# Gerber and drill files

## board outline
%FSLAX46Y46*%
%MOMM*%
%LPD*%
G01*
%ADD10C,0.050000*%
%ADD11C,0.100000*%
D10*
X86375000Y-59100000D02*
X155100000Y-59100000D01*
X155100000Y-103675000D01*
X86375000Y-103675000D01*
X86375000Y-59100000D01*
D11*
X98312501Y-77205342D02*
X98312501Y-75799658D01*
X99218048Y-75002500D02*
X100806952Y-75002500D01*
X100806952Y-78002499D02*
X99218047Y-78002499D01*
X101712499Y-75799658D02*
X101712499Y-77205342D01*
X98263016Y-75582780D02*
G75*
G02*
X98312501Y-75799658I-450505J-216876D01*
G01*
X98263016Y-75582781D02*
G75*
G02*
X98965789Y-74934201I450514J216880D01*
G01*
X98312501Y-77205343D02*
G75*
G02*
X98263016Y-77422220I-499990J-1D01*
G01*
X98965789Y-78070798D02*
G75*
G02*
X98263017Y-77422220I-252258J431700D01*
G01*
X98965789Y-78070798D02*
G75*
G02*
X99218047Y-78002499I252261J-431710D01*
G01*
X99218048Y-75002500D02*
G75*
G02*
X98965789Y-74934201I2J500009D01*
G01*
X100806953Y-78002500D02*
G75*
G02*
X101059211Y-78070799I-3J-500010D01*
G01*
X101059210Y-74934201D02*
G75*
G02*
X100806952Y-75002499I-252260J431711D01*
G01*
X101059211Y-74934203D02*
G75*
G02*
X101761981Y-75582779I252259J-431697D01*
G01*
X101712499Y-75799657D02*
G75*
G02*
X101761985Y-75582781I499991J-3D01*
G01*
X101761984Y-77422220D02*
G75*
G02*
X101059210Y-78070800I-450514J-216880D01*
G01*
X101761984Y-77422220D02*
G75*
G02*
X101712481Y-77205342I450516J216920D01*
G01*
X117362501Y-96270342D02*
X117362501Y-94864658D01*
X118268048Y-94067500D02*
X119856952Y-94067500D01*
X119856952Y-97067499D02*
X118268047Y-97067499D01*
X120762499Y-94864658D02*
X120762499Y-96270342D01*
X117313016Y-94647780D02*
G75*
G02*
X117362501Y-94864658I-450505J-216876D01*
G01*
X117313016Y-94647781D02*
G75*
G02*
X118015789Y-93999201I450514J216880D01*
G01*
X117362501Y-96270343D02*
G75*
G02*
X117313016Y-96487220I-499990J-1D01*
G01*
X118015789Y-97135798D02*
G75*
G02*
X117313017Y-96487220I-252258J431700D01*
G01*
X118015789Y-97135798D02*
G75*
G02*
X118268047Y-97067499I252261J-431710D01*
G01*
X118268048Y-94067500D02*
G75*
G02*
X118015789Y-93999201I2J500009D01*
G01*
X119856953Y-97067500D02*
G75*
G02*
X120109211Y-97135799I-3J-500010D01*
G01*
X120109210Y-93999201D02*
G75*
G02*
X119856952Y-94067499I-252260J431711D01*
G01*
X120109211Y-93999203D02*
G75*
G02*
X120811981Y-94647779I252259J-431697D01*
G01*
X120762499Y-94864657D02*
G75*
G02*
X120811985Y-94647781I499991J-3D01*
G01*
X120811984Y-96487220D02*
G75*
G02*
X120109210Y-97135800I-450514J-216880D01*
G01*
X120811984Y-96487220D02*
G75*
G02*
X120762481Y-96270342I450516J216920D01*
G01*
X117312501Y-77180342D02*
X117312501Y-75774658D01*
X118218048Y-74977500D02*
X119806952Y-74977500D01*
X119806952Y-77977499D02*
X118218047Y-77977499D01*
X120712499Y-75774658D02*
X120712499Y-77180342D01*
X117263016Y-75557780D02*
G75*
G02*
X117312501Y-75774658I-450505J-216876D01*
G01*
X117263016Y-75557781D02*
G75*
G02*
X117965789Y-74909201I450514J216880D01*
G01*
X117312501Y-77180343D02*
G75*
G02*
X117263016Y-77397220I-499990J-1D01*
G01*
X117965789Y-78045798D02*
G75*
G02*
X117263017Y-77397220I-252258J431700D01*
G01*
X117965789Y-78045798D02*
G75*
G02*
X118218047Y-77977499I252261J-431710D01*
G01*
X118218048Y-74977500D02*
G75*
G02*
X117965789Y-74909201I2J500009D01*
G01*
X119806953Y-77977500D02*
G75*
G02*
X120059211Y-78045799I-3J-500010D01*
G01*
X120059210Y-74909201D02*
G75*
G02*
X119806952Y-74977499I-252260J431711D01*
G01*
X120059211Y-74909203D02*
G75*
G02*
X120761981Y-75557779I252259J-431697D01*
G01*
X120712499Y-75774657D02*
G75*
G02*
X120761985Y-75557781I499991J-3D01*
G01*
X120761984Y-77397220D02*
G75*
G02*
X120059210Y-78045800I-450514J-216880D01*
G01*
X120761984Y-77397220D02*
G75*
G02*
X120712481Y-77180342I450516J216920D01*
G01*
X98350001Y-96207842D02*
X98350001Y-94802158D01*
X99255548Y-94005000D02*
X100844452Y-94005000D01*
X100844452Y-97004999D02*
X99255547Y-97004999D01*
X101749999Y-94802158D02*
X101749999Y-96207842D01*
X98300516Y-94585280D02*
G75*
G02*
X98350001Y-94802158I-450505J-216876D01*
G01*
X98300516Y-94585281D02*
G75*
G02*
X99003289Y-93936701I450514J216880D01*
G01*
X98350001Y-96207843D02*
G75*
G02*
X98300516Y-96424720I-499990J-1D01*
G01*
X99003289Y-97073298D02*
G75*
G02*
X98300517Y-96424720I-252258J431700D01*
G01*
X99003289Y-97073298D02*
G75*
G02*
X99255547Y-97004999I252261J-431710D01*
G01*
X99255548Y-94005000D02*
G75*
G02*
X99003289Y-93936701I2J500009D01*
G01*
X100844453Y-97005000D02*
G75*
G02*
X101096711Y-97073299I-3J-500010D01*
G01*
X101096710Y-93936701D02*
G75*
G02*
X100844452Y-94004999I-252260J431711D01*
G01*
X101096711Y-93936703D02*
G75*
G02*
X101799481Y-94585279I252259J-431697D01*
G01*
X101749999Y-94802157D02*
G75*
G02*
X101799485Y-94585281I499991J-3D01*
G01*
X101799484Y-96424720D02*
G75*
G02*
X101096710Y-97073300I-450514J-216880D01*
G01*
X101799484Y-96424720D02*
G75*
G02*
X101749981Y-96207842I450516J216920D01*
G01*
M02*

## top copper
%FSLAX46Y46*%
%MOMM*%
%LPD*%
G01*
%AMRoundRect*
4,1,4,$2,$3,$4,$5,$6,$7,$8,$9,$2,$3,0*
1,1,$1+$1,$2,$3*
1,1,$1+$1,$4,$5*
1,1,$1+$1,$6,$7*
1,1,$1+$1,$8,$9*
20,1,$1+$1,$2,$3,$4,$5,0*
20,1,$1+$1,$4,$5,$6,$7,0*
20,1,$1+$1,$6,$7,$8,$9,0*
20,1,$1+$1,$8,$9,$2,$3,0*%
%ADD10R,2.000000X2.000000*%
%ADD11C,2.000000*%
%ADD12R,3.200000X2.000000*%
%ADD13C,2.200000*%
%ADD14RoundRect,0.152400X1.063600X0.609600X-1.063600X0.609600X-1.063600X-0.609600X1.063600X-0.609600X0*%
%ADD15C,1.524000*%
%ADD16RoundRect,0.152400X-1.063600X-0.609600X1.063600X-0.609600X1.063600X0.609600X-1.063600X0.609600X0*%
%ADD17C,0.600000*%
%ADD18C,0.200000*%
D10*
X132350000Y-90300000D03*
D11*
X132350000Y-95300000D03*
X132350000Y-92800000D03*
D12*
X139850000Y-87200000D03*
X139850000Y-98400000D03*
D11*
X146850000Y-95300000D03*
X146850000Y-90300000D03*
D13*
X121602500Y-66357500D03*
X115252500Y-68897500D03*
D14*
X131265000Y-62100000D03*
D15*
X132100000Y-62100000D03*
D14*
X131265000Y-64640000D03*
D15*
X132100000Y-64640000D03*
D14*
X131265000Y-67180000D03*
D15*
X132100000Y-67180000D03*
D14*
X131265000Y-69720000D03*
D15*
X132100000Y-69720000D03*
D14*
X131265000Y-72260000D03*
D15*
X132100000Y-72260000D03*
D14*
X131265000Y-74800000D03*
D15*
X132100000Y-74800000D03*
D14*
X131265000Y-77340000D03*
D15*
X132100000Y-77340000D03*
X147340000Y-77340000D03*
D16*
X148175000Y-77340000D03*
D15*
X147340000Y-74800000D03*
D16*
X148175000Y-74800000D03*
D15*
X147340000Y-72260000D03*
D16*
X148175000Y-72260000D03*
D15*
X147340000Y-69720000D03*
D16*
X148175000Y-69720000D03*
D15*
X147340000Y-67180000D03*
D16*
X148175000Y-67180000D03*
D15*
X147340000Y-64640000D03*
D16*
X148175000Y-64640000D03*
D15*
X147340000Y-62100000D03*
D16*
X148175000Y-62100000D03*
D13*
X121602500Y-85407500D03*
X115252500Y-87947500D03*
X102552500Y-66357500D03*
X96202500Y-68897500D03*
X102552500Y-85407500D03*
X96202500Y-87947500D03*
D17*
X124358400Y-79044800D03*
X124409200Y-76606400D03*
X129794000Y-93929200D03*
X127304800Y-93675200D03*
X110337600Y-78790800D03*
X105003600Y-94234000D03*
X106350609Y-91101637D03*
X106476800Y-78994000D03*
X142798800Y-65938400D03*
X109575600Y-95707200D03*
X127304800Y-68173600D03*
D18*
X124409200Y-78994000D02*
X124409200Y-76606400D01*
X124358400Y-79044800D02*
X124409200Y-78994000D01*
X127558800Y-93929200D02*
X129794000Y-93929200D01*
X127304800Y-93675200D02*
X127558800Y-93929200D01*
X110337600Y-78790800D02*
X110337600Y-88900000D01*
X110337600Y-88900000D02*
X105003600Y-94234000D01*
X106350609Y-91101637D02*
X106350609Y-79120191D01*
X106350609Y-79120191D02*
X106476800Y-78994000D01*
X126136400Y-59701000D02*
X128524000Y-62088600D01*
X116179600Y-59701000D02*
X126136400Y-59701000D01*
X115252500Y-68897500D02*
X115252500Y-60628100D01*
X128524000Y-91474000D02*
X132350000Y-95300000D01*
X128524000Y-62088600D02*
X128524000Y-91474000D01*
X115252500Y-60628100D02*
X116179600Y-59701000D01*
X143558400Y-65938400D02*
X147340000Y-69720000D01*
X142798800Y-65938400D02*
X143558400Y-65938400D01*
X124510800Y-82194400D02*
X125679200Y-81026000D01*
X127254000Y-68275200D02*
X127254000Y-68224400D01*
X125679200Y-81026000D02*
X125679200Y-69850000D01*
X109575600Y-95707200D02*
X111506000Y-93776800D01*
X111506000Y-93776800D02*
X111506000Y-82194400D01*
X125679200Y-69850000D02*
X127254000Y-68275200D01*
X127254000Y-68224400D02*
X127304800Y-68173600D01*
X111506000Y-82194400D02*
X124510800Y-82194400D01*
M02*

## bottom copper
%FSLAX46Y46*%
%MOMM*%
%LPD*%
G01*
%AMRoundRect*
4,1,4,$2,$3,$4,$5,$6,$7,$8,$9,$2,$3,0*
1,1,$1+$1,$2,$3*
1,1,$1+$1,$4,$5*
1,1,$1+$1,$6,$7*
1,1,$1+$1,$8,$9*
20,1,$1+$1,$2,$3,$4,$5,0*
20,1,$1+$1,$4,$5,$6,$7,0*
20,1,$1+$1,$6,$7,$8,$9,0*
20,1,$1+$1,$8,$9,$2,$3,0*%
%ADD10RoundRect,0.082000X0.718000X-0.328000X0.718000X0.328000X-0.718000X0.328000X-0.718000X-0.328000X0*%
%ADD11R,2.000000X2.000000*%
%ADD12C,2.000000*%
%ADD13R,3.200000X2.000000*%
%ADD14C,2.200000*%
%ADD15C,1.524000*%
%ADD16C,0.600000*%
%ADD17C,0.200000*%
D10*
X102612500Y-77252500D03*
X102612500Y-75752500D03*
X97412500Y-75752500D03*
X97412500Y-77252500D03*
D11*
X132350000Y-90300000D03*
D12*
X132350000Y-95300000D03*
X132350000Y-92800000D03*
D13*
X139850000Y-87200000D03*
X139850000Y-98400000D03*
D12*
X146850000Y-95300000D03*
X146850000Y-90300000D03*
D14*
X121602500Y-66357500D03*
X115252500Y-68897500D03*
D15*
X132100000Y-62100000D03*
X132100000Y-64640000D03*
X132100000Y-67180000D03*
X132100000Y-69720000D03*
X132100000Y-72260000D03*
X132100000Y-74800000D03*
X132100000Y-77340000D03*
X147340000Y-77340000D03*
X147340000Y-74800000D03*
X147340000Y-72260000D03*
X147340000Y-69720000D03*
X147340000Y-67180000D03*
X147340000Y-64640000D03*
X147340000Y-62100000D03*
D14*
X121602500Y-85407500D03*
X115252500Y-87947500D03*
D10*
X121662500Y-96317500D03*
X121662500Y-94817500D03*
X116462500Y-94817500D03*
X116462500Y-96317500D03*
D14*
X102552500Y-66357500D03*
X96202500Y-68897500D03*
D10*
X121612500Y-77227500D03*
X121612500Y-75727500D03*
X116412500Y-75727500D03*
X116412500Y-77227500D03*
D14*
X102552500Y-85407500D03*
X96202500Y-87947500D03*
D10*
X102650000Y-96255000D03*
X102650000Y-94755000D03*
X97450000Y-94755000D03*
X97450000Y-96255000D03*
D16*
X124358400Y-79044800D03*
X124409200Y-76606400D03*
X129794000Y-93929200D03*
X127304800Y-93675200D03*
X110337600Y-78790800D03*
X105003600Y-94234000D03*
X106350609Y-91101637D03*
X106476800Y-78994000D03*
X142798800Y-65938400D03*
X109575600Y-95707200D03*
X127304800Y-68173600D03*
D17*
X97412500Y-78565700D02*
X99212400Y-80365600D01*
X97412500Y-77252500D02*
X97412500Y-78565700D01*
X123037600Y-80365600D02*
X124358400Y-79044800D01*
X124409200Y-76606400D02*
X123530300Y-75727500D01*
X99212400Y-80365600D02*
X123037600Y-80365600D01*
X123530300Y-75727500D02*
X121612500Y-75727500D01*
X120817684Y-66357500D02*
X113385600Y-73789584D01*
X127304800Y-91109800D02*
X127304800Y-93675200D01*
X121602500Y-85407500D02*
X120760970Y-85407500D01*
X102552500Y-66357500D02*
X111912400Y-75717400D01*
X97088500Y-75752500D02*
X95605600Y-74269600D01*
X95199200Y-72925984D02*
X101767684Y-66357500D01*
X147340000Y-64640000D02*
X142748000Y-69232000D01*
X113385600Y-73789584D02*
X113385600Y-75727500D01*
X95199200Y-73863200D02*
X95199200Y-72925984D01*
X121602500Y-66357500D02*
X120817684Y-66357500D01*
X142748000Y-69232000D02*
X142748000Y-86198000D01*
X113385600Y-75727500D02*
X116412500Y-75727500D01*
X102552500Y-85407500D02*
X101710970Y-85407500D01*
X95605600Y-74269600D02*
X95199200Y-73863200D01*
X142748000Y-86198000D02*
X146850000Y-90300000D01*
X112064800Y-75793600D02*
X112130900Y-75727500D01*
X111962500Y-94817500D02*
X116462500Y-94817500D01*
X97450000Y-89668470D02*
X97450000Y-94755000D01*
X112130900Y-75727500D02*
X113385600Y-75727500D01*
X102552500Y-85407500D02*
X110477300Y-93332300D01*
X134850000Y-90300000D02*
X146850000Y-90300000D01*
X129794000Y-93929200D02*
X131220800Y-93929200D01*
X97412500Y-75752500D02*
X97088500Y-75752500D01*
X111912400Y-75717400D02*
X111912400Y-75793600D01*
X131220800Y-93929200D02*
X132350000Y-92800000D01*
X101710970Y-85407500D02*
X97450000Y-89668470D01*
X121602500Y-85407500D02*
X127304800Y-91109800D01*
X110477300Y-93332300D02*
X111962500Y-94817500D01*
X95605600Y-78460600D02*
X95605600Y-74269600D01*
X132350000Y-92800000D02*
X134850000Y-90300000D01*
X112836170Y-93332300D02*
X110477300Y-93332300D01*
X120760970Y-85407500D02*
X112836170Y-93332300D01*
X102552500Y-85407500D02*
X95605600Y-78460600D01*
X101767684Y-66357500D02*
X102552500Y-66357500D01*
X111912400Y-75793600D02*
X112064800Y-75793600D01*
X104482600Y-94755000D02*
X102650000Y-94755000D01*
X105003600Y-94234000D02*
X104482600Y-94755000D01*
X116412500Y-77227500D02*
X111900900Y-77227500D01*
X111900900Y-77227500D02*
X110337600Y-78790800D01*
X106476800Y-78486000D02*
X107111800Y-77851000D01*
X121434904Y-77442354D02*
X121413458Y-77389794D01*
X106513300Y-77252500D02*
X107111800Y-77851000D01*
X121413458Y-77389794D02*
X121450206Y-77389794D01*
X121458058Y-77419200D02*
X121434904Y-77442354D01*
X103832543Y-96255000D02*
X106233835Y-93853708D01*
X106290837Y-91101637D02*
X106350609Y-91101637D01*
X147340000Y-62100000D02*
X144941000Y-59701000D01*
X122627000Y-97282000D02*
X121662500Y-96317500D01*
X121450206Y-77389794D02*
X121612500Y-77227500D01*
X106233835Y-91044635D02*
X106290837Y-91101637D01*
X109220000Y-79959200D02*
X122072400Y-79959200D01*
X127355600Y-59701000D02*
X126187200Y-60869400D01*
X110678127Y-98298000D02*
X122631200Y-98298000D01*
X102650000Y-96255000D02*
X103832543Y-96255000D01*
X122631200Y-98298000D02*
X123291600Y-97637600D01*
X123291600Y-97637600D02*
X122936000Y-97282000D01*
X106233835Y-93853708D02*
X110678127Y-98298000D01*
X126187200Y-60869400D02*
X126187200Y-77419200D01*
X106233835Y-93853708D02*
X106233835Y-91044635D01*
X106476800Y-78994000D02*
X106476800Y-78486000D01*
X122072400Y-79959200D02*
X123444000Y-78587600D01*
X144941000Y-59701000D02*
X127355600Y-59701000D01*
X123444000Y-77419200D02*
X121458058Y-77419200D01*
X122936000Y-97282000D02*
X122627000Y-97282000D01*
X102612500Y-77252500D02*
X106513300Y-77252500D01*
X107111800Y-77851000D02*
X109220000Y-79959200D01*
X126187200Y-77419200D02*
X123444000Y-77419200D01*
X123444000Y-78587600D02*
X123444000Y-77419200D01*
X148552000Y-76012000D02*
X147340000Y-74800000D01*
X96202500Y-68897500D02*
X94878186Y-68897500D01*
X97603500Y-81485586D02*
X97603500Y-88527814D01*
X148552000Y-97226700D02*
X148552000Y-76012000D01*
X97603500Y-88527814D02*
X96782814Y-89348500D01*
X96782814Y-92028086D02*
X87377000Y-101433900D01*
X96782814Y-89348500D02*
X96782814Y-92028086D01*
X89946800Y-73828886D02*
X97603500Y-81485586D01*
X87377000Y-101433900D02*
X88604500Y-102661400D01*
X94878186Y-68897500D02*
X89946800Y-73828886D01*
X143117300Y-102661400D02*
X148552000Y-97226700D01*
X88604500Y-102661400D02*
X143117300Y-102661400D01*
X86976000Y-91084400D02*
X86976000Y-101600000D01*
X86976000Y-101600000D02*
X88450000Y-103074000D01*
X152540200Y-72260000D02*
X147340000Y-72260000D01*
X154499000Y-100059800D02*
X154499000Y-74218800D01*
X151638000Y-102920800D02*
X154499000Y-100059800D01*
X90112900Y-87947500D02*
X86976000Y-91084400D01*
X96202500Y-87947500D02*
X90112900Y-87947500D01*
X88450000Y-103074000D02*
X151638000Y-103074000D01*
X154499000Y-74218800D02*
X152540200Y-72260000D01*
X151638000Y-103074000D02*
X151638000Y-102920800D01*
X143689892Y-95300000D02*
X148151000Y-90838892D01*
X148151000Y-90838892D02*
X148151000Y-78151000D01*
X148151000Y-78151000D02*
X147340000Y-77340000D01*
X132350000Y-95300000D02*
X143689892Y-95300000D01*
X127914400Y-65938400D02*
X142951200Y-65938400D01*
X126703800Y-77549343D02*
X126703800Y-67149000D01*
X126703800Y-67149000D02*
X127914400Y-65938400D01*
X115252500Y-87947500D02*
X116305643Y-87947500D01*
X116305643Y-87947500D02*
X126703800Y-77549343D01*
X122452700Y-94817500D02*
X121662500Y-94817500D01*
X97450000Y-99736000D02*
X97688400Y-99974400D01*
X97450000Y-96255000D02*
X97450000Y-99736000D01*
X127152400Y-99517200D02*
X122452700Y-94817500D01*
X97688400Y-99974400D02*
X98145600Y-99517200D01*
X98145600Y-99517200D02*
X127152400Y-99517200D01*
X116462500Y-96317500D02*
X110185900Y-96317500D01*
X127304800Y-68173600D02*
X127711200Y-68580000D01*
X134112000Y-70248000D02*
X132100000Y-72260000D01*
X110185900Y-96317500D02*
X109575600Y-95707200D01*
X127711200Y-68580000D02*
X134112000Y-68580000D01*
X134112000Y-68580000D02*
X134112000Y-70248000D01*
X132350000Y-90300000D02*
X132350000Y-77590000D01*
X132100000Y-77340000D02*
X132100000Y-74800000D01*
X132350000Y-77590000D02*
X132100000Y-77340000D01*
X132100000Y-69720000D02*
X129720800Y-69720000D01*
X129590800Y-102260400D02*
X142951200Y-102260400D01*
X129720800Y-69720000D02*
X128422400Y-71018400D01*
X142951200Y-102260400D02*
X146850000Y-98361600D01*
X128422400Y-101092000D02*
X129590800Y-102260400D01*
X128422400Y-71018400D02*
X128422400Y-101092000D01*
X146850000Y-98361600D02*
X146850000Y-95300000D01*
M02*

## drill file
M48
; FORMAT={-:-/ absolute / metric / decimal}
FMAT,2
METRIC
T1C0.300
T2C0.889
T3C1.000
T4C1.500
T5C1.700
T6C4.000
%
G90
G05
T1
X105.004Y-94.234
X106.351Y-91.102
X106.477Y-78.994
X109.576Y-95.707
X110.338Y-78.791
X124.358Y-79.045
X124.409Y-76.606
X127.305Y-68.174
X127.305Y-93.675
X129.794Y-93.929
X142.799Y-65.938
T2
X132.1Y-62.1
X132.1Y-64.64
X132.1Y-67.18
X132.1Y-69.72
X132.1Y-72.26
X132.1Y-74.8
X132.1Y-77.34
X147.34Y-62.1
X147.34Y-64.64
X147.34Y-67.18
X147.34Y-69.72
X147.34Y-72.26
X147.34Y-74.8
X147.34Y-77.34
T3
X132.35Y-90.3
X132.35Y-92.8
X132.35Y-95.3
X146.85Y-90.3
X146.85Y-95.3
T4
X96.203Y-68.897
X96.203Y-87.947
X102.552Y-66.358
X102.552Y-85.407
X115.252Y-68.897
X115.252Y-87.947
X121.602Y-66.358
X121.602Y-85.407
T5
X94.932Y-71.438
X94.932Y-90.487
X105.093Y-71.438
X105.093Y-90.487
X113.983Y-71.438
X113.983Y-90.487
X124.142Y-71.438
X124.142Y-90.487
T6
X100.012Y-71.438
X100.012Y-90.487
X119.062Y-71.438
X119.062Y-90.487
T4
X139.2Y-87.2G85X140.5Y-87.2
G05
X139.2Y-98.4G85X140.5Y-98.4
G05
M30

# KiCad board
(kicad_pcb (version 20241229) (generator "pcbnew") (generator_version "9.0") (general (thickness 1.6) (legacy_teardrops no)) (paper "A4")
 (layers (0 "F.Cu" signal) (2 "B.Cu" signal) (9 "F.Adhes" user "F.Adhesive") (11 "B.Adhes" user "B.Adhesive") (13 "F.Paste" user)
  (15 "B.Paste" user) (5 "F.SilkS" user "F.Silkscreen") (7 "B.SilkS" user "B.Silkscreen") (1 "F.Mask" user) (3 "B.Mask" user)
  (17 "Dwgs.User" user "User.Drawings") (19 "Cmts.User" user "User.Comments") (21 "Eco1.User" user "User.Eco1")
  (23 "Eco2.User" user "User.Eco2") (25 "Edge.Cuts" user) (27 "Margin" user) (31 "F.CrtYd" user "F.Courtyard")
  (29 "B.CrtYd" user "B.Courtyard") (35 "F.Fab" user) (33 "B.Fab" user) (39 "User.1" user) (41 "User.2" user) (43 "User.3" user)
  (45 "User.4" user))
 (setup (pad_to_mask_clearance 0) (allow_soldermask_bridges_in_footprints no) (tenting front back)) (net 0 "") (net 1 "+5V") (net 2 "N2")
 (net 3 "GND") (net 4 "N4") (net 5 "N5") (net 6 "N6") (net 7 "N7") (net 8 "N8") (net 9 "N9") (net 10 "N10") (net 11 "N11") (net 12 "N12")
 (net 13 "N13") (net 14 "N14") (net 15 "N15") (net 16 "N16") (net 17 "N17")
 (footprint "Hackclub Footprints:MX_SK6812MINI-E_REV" (layer "F.Cu") (at 100.0125 71.4225)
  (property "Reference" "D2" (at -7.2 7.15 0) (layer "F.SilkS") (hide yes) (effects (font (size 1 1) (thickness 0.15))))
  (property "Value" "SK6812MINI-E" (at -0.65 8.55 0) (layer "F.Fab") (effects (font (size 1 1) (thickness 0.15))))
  (fp_line (start -1.699999 5.782842) (end -1.699999 4.377158) (stroke (width 0.1) (type solid)) (layer "Edge.Cuts"))
  (fp_line (start -0.794452 3.58) (end 0.794452 3.58) (stroke (width 0.1) (type solid)) (layer "Edge.Cuts"))
  (fp_line (start 0.794452 6.579999) (end -0.794453 6.579999) (stroke (width 0.1) (type solid)) (layer "Edge.Cuts"))
  (fp_line (start 1.699999 4.377158) (end 1.699999 5.782842) (stroke (width 0.1) (type solid)) (layer "Edge.Cuts"))
  (fp_arc (start -1.749484 4.16028) (mid -1.712527 4.265932) (end -1.699999 4.377158) (stroke (width 0.1) (type solid)) (layer "Edge.Cuts"))
  (fp_arc (start -1.749484 4.160281) (mid -1.638072 3.575965) (end -1.046711 3.511701) (stroke (width 0.1) (type solid)) (layer "Edge.Cuts"))
  (fp_arc (start -1.699999 5.782843) (mid -1.712527 5.894068) (end -1.749484 5.99972) (stroke (width 0.1) (type solid)) (layer "Edge.Cuts"))
  (fp_arc (start -1.046711 6.648298) (mid -1.638071 6.584034) (end -1.749484 5.99972) (stroke (width 0.1) (type solid)) (layer "Edge.Cuts"))
  (fp_arc (start -1.046711 6.648298) (mid -0.925123 6.597376) (end -0.794453 6.579999) (stroke (width 0.1) (type solid)) (layer "Edge.Cuts"))
  (fp_arc (start -0.794452 3.58) (mid -0.925123 3.562623) (end -1.046711 3.511701) (stroke (width 0.1) (type solid)) (layer "Edge.Cuts"))
  (fp_arc (start 0.794453 6.58) (mid 0.925123 6.597377) (end 1.046711 6.648299) (stroke (width 0.1) (type solid)) (layer "Edge.Cuts"))
  (fp_arc (start 1.04671 3.511701) (mid 0.925122 3.562623) (end 0.794452 3.58) (stroke (width 0.1) (type solid)) (layer "Edge.Cuts"))
  (fp_arc (start 1.046711 3.511703) (mid 1.63807 3.575966) (end 1.749484 4.16028) (stroke (width 0.1) (type solid)) (layer "Edge.Cuts"))
  (fp_arc (start 1.699999 4.377157) (mid 1.712527 4.265932) (end 1.749484 4.16028) (stroke (width 0.1) (type solid)) (layer "Edge.Cuts"))
  (fp_arc (start 1.749484 5.99972) (mid 1.638071 6.584035) (end 1.046711 6.648299) (stroke (width 0.1) (type solid)) (layer "Edge.Cuts"))
  (fp_arc (start 1.749484 5.99972) (mid 1.712527 5.894068) (end 1.699999 5.782842) (stroke (width 0.1) (type solid)) (layer "Edge.Cuts"))
  (pad "1" smd roundrect (at 2.6 5.83 90) (size 0.82 1.6) (layers "B.Cu" "B.Mask" "B.Paste") (roundrect_rratio 0.1) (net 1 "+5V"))
  (pad "2" smd roundrect (at 2.6 4.33 90) (size 0.82 1.6) (layers "B.Cu" "B.Mask" "B.Paste") (roundrect_rratio 0.1) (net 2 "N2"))
  (pad "3" smd roundrect (at -2.6 4.33 90) (size 0.82 1.6) (layers "B.Cu" "B.Mask" "B.Paste") (roundrect_rratio 0.1) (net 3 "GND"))
  (pad "4" smd roundrect (at -2.6 5.83 90) (size 0.82 1.6) (layers "B.Cu" "B.Mask" "B.Paste") (roundrect_rratio 0.1) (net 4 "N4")))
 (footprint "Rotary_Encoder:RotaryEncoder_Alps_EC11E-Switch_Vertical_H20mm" (layer "F.Cu") (at 132.35 90.3)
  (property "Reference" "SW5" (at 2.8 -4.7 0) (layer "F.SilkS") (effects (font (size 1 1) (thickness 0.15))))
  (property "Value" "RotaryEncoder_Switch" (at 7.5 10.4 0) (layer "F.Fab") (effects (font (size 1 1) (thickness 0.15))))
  (pad "A" thru_hole rect (at 0 0) (size 2 2) (drill 1) (layers "*.Cu" "*.Mask") (remove_unused_layers no) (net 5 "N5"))
  (pad "B" thru_hole circle (at 0 5) (size 2 2) (drill 1) (layers "*.Cu" "*.Mask") (remove_unused_layers no) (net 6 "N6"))
  (pad "C" thru_hole circle (at 0 2.5) (size 2 2) (drill 1) (layers "*.Cu" "*.Mask") (remove_unused_layers no) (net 3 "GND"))
  (pad "MP" thru_hole rect (at 7.5 -3.1) (size 3.2 2) (drill oval 2.8 1.5) (layers "*.Cu" "*.Mask") (remove_unused_layers no))
  (pad "MP" thru_hole rect (at 7.5 8.1) (size 3.2 2) (drill oval 2.8 1.5) (layers "*.Cu" "*.Mask") (remove_unused_layers no))
  (pad "S1" thru_hole circle (at 14.5 5) (size 2 2) (drill 1) (layers "*.Cu" "*.Mask") (remove_unused_layers no) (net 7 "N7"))
  (pad "S2" thru_hole circle (at 14.5 0) (size 2 2) (drill 1) (layers "*.Cu" "*.Mask") (remove_unused_layers no) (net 3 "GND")))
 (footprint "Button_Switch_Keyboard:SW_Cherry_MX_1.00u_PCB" (layer "F.Cu") (at 121.6025 66.3575)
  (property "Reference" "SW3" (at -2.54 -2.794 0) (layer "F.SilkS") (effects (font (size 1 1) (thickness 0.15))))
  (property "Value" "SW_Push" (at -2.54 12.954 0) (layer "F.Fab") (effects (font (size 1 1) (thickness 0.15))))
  (pad "" np_thru_hole circle (at -7.62 5.08) (size 1.7 1.7) (drill 1.7) (layers "*.Cu" "*.Mask"))
  (pad "" np_thru_hole circle (at -2.54 5.08) (size 4 4) (drill 4) (layers "*.Cu" "*.Mask"))
  (pad "" np_thru_hole circle (at 2.54 5.08) (size 1.7 1.7) (drill 1.7) (layers "*.Cu" "*.Mask"))
  (pad "1" thru_hole circle (at 0 0) (size 2.2 2.2) (drill 1.5) (layers "*.Cu" "*.Mask") (remove_unused_layers no) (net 3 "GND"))
  (pad "2" thru_hole circle (at -6.35 2.54) (size 2.2 2.2) (drill 1.5) (layers "*.Cu" "*.Mask") (remove_unused_layers no) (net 6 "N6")))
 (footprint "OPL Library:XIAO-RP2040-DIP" (layer "F.Cu") (at 139.72 69.72)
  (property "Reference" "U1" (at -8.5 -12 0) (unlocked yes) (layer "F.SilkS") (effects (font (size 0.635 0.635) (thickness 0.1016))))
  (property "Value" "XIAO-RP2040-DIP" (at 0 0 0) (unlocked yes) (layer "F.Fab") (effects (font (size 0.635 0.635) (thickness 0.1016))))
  (pad "1" smd roundrect (at -8.455 -7.62 180) (size 2.432 1.524) (layers "F.Cu" "F.Mask") (roundrect_rratio 0.1) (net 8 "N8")
   (thermal_bridge_angle 45))
  (pad "1" thru_hole circle (at -7.62 -7.62 180) (size 1.524 1.524) (drill 0.889) (layers "*.Cu" "*.Mask") (remove_unused_layers no)
   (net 8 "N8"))
  (pad "2" smd roundrect (at -8.455 -5.08 180) (size 2.432 1.524) (layers "F.Cu" "F.Mask") (roundrect_rratio 0.1) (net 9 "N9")
   (thermal_bridge_angle 45))
  (pad "2" thru_hole circle (at -7.62 -5.08 180) (size 1.524 1.524) (drill 0.889) (layers "*.Cu" "*.Mask") (remove_unused_layers no)
   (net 9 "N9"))
  (pad "3" smd roundrect (at -8.455 -2.54 180) (size 2.432 1.524) (layers "F.Cu" "F.Mask") (roundrect_rratio 0.1) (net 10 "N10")
   (thermal_bridge_angle 45))
  (pad "3" thru_hole circle (at -7.62 -2.54 180) (size 1.524 1.524) (drill 0.889) (layers "*.Cu" "*.Mask") (remove_unused_layers no)
   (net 10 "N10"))
  (pad "4" smd roundrect (at -8.455 0 180) (size 2.432 1.524) (layers "F.Cu" "F.Mask") (roundrect_rratio 0.1) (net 7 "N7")
   (thermal_bridge_angle 45))
  (pad "4" thru_hole circle (at -7.62 0 180) (size 1.524 1.524) (drill 0.889) (layers "*.Cu" "*.Mask") (remove_unused_layers no)
   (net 7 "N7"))
  (pad "5" smd roundrect (at -8.455 2.54 180) (size 2.432 1.524) (layers "F.Cu" "F.Mask") (roundrect_rratio 0.1) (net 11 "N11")
   (thermal_bridge_angle 45))
  (pad "5" thru_hole circle (at -7.62 2.54 180) (size 1.524 1.524) (drill 0.889) (layers "*.Cu" "*.Mask") (remove_unused_layers no)
   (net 11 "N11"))
  (pad "6" smd roundrect (at -8.455 5.08 180) (size 2.432 1.524) (layers "F.Cu" "F.Mask") (roundrect_rratio 0.1) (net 5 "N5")
   (thermal_bridge_angle 45))
  (pad "6" thru_hole circle (at -7.62 5.08 180) (size 1.524 1.524) (drill 0.889) (layers "*.Cu" "*.Mask") (remove_unused_layers no)
   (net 5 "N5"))
  (pad "7" smd roundrect (at -8.455 7.62 180) (size 2.432 1.524) (layers "F.Cu" "F.Mask") (roundrect_rratio 0.1) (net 5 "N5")
   (thermal_bridge_angle 45))
  (pad "7" thru_hole circle (at -7.62 7.62 180) (size 1.524 1.524) (drill 0.889) (layers "*.Cu" "*.Mask") (remove_unused_layers no)
   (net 5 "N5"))
  (pad "8" thru_hole circle (at 7.62 7.62) (size 1.524 1.524) (drill 0.889) (layers "*.Cu" "*.Mask") (remove_unused_layers no) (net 6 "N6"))
  (pad "8" smd roundrect (at 8.455 7.62) (size 2.432 1.524) (layers "F.Cu" "F.Mask") (roundrect_rratio 0.1) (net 6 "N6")
   (thermal_bridge_angle 45))
  (pad "9" thru_hole circle (at 7.62 5.08) (size 1.524 1.524) (drill 0.889) (layers "*.Cu" "*.Mask") (remove_unused_layers no)
   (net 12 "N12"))
  (pad "9" smd roundrect (at 8.455 5.08) (size 2.432 1.524) (layers "F.Cu" "F.Mask") (roundrect_rratio 0.1) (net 12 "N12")
   (thermal_bridge_angle 45))
  (pad "10" thru_hole circle (at 7.62 2.54) (size 1.524 1.524) (drill 0.889) (layers "*.Cu" "*.Mask") (remove_unused_layers no)
   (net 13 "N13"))
  (pad "10" smd roundrect (at 8.455 2.54) (size 2.432 1.524) (layers "F.Cu" "F.Mask") (roundrect_rratio 0.1) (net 13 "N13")
   (thermal_bridge_angle 45))
  (pad "11" thru_hole circle (at 7.62 0) (size 1.524 1.524) (drill 0.889) (layers "*.Cu" "*.Mask") (remove_unused_layers no) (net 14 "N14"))
  (pad "11" smd roundrect (at 8.455 0) (size 2.432 1.524) (layers "F.Cu" "F.Mask") (roundrect_rratio 0.1) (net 14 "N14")
   (thermal_bridge_angle 45))
  (pad "12" thru_hole circle (at 7.62 -2.54) (size 1.524 1.524) (drill 0.889) (layers "*.Cu" "*.Mask") (remove_unused_layers no)
   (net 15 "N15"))
  (pad "12" smd roundrect (at 8.455 -2.54) (size 2.432 1.524) (layers "F.Cu" "F.Mask") (roundrect_rratio 0.1) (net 15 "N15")
   (thermal_bridge_angle 45))
  (pad "13" thru_hole circle (at 7.62 -5.08) (size 1.524 1.524) (drill 0.889) (layers "*.Cu" "*.Mask") (remove_unused_layers no)
   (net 3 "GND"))
  (pad "13" smd roundrect (at 8.455 -5.08) (size 2.432 1.524) (layers "F.Cu" "F.Mask") (roundrect_rratio 0.1) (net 3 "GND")
   (thermal_bridge_angle 45))
  (pad "14" thru_hole circle (at 7.62 -7.62) (size 1.524 1.524) (drill 0.889) (layers "*.Cu" "*.Mask") (remove_unused_layers no)
   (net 1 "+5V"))
  (pad "14" smd roundrect (at 8.455 -7.62) (size 2.432 1.524) (layers "F.Cu" "F.Mask") (roundrect_rratio 0.1) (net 1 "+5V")
   (thermal_bridge_angle 45)))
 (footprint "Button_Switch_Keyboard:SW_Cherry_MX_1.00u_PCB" (layer "F.Cu") (at 121.6025 85.4075)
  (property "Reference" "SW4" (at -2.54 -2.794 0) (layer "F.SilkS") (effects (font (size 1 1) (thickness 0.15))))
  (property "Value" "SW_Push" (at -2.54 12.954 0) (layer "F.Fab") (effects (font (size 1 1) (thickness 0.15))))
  (pad "" np_thru_hole circle (at -7.62 5.08) (size 1.7 1.7) (drill 1.7) (layers "*.Cu" "*.Mask"))
  (pad "" np_thru_hole circle (at -2.54 5.08) (size 4 4) (drill 4) (layers "*.Cu" "*.Mask"))
  (pad "" np_thru_hole circle (at 2.54 5.08) (size 1.7 1.7) (drill 1.7) (layers "*.Cu" "*.Mask"))
  (pad "1" thru_hole circle (at 0 0) (size 2.2 2.2) (drill 1.5) (layers "*.Cu" "*.Mask") (remove_unused_layers no) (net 3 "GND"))
  (pad "2" thru_hole circle (at -6.35 2.54) (size 2.2 2.2) (drill 1.5) (layers "*.Cu" "*.Mask") (remove_unused_layers no) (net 14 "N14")))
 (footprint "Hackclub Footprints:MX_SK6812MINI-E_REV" (layer "F.Cu") (at 119.0625 90.4875)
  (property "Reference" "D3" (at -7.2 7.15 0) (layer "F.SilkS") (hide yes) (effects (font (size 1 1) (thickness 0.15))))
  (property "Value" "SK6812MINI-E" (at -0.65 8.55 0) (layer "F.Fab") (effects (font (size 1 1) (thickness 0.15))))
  (fp_line (start -1.699999 5.782842) (end -1.699999 4.377158) (stroke (width 0.1) (type solid)) (layer "Edge.Cuts"))
  (fp_line (start -0.794452 3.58) (end 0.794452 3.58) (stroke (width 0.1) (type solid)) (layer "Edge.Cuts"))
  (fp_line (start 0.794452 6.579999) (end -0.794453 6.579999) (stroke (width 0.1) (type solid)) (layer "Edge.Cuts"))
  (fp_line (start 1.699999 4.377158) (end 1.699999 5.782842) (stroke (width 0.1) (type solid)) (layer "Edge.Cuts"))
  (fp_arc (start -1.749484 4.16028) (mid -1.712527 4.265932) (end -1.699999 4.377158) (stroke (width 0.1) (type solid)) (layer "Edge.Cuts"))
  (fp_arc (start -1.749484 4.160281) (mid -1.638072 3.575965) (end -1.046711 3.511701) (stroke (width 0.1) (type solid)) (layer "Edge.Cuts"))
  (fp_arc (start -1.699999 5.782843) (mid -1.712527 5.894068) (end -1.749484 5.99972) (stroke (width 0.1) (type solid)) (layer "Edge.Cuts"))
  (fp_arc (start -1.046711 6.648298) (mid -1.638071 6.584034) (end -1.749484 5.99972) (stroke (width 0.1) (type solid)) (layer "Edge.Cuts"))
  (fp_arc (start -1.046711 6.648298) (mid -0.925123 6.597376) (end -0.794453 6.579999) (stroke (width 0.1) (type solid)) (layer "Edge.Cuts"))
  (fp_arc (start -0.794452 3.58) (mid -0.925123 3.562623) (end -1.046711 3.511701) (stroke (width 0.1) (type solid)) (layer "Edge.Cuts"))
  (fp_arc (start 0.794453 6.58) (mid 0.925123 6.597377) (end 1.046711 6.648299) (stroke (width 0.1) (type solid)) (layer "Edge.Cuts"))
  (fp_arc (start 1.04671 3.511701) (mid 0.925122 3.562623) (end 0.794452 3.58) (stroke (width 0.1) (type solid)) (layer "Edge.Cuts"))
  (fp_arc (start 1.046711 3.511703) (mid 1.63807 3.575966) (end 1.749484 4.16028) (stroke (width 0.1) (type solid)) (layer "Edge.Cuts"))
  (fp_arc (start 1.699999 4.377157) (mid 1.712527 4.265932) (end 1.749484 4.16028) (stroke (width 0.1) (type solid)) (layer "Edge.Cuts"))
  (fp_arc (start 1.749484 5.99972) (mid 1.638071 6.584035) (end 1.046711 6.648299) (stroke (width 0.1) (type solid)) (layer "Edge.Cuts"))
  (fp_arc (start 1.749484 5.99972) (mid 1.712527 5.894068) (end 1.699999 5.782842) (stroke (width 0.1) (type solid)) (layer "Edge.Cuts"))
  (pad "1" smd roundrect (at 2.6 5.83 90) (size 0.82 1.6) (layers "B.Cu" "B.Mask" "B.Paste") (roundrect_rratio 0.1) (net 1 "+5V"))
  (pad "2" smd roundrect (at 2.6 4.33 90) (size 0.82 1.6) (layers "B.Cu" "B.Mask" "B.Paste") (roundrect_rratio 0.1) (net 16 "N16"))
  (pad "3" smd roundrect (at -2.6 4.33 90) (size 0.82 1.6) (layers "B.Cu" "B.Mask" "B.Paste") (roundrect_rratio 0.1) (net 3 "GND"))
  (pad "4" smd roundrect (at -2.6 5.83 90) (size 0.82 1.6) (layers "B.Cu" "B.Mask" "B.Paste") (roundrect_rratio 0.1) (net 11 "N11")))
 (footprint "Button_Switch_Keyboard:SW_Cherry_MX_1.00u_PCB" (layer "F.Cu") (at 102.5525 66.3575)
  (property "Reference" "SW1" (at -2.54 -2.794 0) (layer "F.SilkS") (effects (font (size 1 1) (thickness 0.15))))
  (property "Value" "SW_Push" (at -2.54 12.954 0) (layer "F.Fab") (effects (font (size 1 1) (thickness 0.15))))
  (pad "" np_thru_hole circle (at -7.62 5.08) (size 1.7 1.7) (drill 1.7) (layers "*.Cu" "*.Mask"))
  (pad "" np_thru_hole circle (at -2.54 5.08) (size 4 4) (drill 4) (layers "*.Cu" "*.Mask"))
  (pad "" np_thru_hole circle (at 2.54 5.08) (size 1.7 1.7) (drill 1.7) (layers "*.Cu" "*.Mask"))
  (pad "1" thru_hole circle (at 0 0) (size 2.2 2.2) (drill 1.5) (layers "*.Cu" "*.Mask") (remove_unused_layers no) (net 3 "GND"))
  (pad "2" thru_hole circle (at -6.35 2.54) (size 2.2 2.2) (drill 1.5) (layers "*.Cu" "*.Mask") (remove_unused_layers no) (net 12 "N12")))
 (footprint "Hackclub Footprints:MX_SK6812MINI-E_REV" (layer "F.Cu") (at 119.0125 71.3975)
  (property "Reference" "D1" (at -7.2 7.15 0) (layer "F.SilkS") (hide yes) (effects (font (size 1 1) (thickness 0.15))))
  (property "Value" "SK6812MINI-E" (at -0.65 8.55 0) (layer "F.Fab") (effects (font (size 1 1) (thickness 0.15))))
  (fp_line (start -1.699999 5.782842) (end -1.699999 4.377158) (stroke (width 0.1) (type solid)) (layer "Edge.Cuts"))
  (fp_line (start -0.794452 3.58) (end 0.794452 3.58) (stroke (width 0.1) (type solid)) (layer "Edge.Cuts"))
  (fp_line (start 0.794452 6.579999) (end -0.794453 6.579999) (stroke (width 0.1) (type solid)) (layer "Edge.Cuts"))
  (fp_line (start 1.699999 4.377158) (end 1.699999 5.782842) (stroke (width 0.1) (type solid)) (layer "Edge.Cuts"))
  (fp_arc (start -1.749484 4.16028) (mid -1.712527 4.265932) (end -1.699999 4.377158) (stroke (width 0.1) (type solid)) (layer "Edge.Cuts"))
  (fp_arc (start -1.749484 4.160281) (mid -1.638072 3.575965) (end -1.046711 3.511701) (stroke (width 0.1) (type solid)) (layer "Edge.Cuts"))
  (fp_arc (start -1.699999 5.782843) (mid -1.712527 5.894068) (end -1.749484 5.99972) (stroke (width 0.1) (type solid)) (layer "Edge.Cuts"))
  (fp_arc (start -1.046711 6.648298) (mid -1.638071 6.584034) (end -1.749484 5.99972) (stroke (width 0.1) (type solid)) (layer "Edge.Cuts"))
  (fp_arc (start -1.046711 6.648298) (mid -0.925123 6.597376) (end -0.794453 6.579999) (stroke (width 0.1) (type solid)) (layer "Edge.Cuts"))
  (fp_arc (start -0.794452 3.58) (mid -0.925123 3.562623) (end -1.046711 3.511701) (stroke (width 0.1) (type solid)) (layer "Edge.Cuts"))
  (fp_arc (start 0.794453 6.58) (mid 0.925123 6.597377) (end 1.046711 6.648299) (stroke (width 0.1) (type solid)) (layer "Edge.Cuts"))
  (fp_arc (start 1.04671 3.511701) (mid 0.925122 3.562623) (end 0.794452 3.58) (stroke (width 0.1) (type solid)) (layer "Edge.Cuts"))
  (fp_arc (start 1.046711 3.511703) (mid 1.63807 3.575966) (end 1.749484 4.16028) (stroke (width 0.1) (type solid)) (layer "Edge.Cuts"))
  (fp_arc (start 1.699999 4.377157) (mid 1.712527 4.265932) (end 1.749484 4.16028) (stroke (width 0.1) (type solid)) (layer "Edge.Cuts"))
  (fp_arc (start 1.749484 5.99972) (mid 1.638071 6.584035) (end 1.046711 6.648299) (stroke (width 0.1) (type solid)) (layer "Edge.Cuts"))
  (fp_arc (start 1.749484 5.99972) (mid 1.712527 5.894068) (end 1.699999 5.782842) (stroke (width 0.1) (type solid)) (layer "Edge.Cuts"))
  (pad "1" smd roundrect (at 2.6 5.83 90) (size 0.82 1.6) (layers "B.Cu" "B.Mask" "B.Paste") (roundrect_rratio 0.1) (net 1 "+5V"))
  (pad "2" smd roundrect (at 2.6 4.33 90) (size 0.82 1.6) (layers "B.Cu" "B.Mask" "B.Paste") (roundrect_rratio 0.1) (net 4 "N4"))
  (pad "3" smd roundrect (at -2.6 4.33 90) (size 0.82 1.6) (layers "B.Cu" "B.Mask" "B.Paste") (roundrect_rratio 0.1) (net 3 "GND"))
  (pad "4" smd roundrect (at -2.6 5.83 90) (size 0.82 1.6) (layers "B.Cu" "B.Mask" "B.Paste") (roundrect_rratio 0.1) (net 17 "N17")))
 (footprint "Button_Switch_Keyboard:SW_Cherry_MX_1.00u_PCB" (layer "F.Cu") (at 102.5525 85.4075)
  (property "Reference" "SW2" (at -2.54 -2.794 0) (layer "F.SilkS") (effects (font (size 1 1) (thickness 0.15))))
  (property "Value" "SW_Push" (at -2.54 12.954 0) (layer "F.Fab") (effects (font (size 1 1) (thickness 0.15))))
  (pad "" np_thru_hole circle (at -7.62 5.08) (size 1.7 1.7) (drill 1.7) (layers "*.Cu" "*.Mask"))
  (pad "" np_thru_hole circle (at -2.54 5.08) (size 4 4) (drill 4) (layers "*.Cu" "*.Mask"))
  (pad "" np_thru_hole circle (at 2.54 5.08) (size 1.7 1.7) (drill 1.7) (layers "*.Cu" "*.Mask"))
  (pad "1" thru_hole circle (at 0 0) (size 2.2 2.2) (drill 1.5) (layers "*.Cu" "*.Mask") (remove_unused_layers no) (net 3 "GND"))
  (pad "2" thru_hole circle (at -6.35 2.54) (size 2.2 2.2) (drill 1.5) (layers "*.Cu" "*.Mask") (remove_unused_layers no) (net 13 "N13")))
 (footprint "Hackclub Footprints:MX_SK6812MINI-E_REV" (layer "F.Cu") (at 100.05 90.425)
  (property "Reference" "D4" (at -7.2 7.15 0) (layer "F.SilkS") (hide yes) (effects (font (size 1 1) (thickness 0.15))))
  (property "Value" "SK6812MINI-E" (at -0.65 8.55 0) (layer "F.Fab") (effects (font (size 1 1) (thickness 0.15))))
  (fp_line (start -1.699999 5.782842) (end -1.699999 4.377158) (stroke (width 0.1) (type solid)) (layer "Edge.Cuts"))
  (fp_line (start -0.794452 3.58) (end 0.794452 3.58) (stroke (width 0.1) (type solid)) (layer "Edge.Cuts"))
  (fp_line (start 0.794452 6.579999) (end -0.794453 6.579999) (stroke (width 0.1) (type solid)) (layer "Edge.Cuts"))
  (fp_line (start 1.699999 4.377158) (end 1.699999 5.782842) (stroke (width 0.1) (type solid)) (layer "Edge.Cuts"))
  (fp_arc (start -1.749484 4.16028) (mid -1.712527 4.265932) (end -1.699999 4.377158) (stroke (width 0.1) (type solid)) (layer "Edge.Cuts"))
  (fp_arc (start -1.749484 4.160281) (mid -1.638072 3.575965) (end -1.046711 3.511701) (stroke (width 0.1) (type solid)) (layer "Edge.Cuts"))
  (fp_arc (start -1.699999 5.782843) (mid -1.712527 5.894068) (end -1.749484 5.99972) (stroke (width 0.1) (type solid)) (layer "Edge.Cuts"))
  (fp_arc (start -1.046711 6.648298) (mid -1.638071 6.584034) (end -1.749484 5.99972) (stroke (width 0.1) (type solid)) (layer "Edge.Cuts"))
  (fp_arc (start -1.046711 6.648298) (mid -0.925123 6.597376) (end -0.794453 6.579999) (stroke (width 0.1) (type solid)) (layer "Edge.Cuts"))
  (fp_arc (start -0.794452 3.58) (mid -0.925123 3.562623) (end -1.046711 3.511701) (stroke (width 0.1) (type solid)) (layer "Edge.Cuts"))
  (fp_arc (start 0.794453 6.58) (mid 0.925123 6.597377) (end 1.046711 6.648299) (stroke (width 0.1) (type solid)) (layer "Edge.Cuts"))
  (fp_arc (start 1.04671 3.511701) (mid 0.925122 3.562623) (end 0.794452 3.58) (stroke (width 0.1) (type solid)) (layer "Edge.Cuts"))
  (fp_arc (start 1.046711 3.511703) (mid 1.63807 3.575966) (end 1.749484 4.16028) (stroke (width 0.1) (type solid)) (layer "Edge.Cuts"))
  (fp_arc (start 1.699999 4.377157) (mid 1.712527 4.265932) (end 1.749484 4.16028) (stroke (width 0.1) (type solid)) (layer "Edge.Cuts"))
  (fp_arc (start 1.749484 5.99972) (mid 1.638071 6.584035) (end 1.046711 6.648299) (stroke (width 0.1) (type solid)) (layer "Edge.Cuts"))
  (fp_arc (start 1.749484 5.99972) (mid 1.712527 5.894068) (end 1.699999 5.782842) (stroke (width 0.1) (type solid)) (layer "Edge.Cuts"))
  (pad "1" smd roundrect (at 2.6 5.83 90) (size 0.82 1.6) (layers "B.Cu" "B.Mask" "B.Paste") (roundrect_rratio 0.1) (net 1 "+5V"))
  (pad "2" smd roundrect (at 2.6 4.33 90) (size 0.82 1.6) (layers "B.Cu" "B.Mask" "B.Paste") (roundrect_rratio 0.1) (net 17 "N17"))
  (pad "3" smd roundrect (at -2.6 4.33 90) (size 0.82 1.6) (layers "B.Cu" "B.Mask" "B.Paste") (roundrect_rratio 0.1) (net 3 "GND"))
  (pad "4" smd roundrect (at -2.6 5.83 90) (size 0.82 1.6) (layers "B.Cu" "B.Mask" "B.Paste") (roundrect_rratio 0.1) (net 16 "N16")))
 (gr_rect (start 86.375 59.1) (end 155.1 103.675) (stroke (width 0.05) (type default)) (fill no) (layer "Edge.Cuts"))
 (segment (start 124.4092 78.994) (end 124.4092 76.6064) (width 0.2) (layer "F.Cu") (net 4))
 (segment (start 124.3584 79.0448) (end 124.4092 78.994) (width 0.2) (layer "F.Cu") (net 4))
 (via (at 124.3584 79.0448) (size 0.6) (drill 0.3) (layers "F.Cu" "B.Cu") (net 4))
 (via (at 124.4092 76.6064) (size 0.6) (drill 0.3) (layers "F.Cu" "B.Cu") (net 4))
 (segment (start 97.4125 78.5657) (end 99.2124 80.3656) (width 0.2) (layer "B.Cu") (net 4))
 (segment (start 97.4125 77.2525) (end 97.4125 78.5657) (width 0.2) (layer "B.Cu") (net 4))
 (segment (start 123.0376 80.3656) (end 124.3584 79.0448) (width 0.2) (layer "B.Cu") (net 4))
 (segment (start 124.4092 76.6064) (end 123.5303 75.7275) (width 0.2) (layer "B.Cu") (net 4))
 (segment (start 99.2124 80.3656) (end 123.0376 80.3656) (width 0.2) (layer "B.Cu") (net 4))
 (segment (start 123.5303 75.7275) (end 121.6125 75.7275) (width 0.2) (layer "B.Cu") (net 4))
 (segment (start 127.5588 93.9292) (end 129.794 93.9292) (width 0.2) (layer "F.Cu") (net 3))
 (segment (start 127.3048 93.6752) (end 127.5588 93.9292) (width 0.2) (layer "F.Cu") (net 3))
 (via (at 129.794 93.9292) (size 0.6) (drill 0.3) (layers "F.Cu" "B.Cu") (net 3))
 (via (at 127.3048 93.6752) (size 0.6) (drill 0.3) (layers "F.Cu" "B.Cu") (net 3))
 (segment (start 120.817684 66.3575) (end 113.3856 73.789584) (width 0.2) (layer "B.Cu") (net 3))
 (segment (start 127.3048 91.1098) (end 127.3048 93.6752) (width 0.2) (layer "B.Cu") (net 3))
 (segment (start 121.6025 85.4075) (end 120.76097 85.4075) (width 0.2) (layer "B.Cu") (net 3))
 (segment (start 102.5525 66.3575) (end 111.9124 75.7174) (width 0.2) (layer "B.Cu") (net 3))
 (segment (start 97.0885 75.7525) (end 95.6056 74.2696) (width 0.2) (layer "B.Cu") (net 3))
 (segment (start 95.1992 72.925984) (end 101.767684 66.3575) (width 0.2) (layer "B.Cu") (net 3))
 (segment (start 147.34 64.64) (end 142.748 69.232) (width 0.2) (layer "B.Cu") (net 3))
 (segment (start 113.3856 73.789584) (end 113.3856 75.7275) (width 0.2) (layer "B.Cu") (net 3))
 (segment (start 95.1992 73.8632) (end 95.1992 72.925984) (width 0.2) (layer "B.Cu") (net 3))
 (segment (start 121.6025 66.3575) (end 120.817684 66.3575) (width 0.2) (layer "B.Cu") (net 3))
 (segment (start 142.748 69.232) (end 142.748 86.198) (width 0.2) (layer "B.Cu") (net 3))
 (segment (start 113.3856 75.7275) (end 116.4125 75.7275) (width 0.2) (layer "B.Cu") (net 3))
 (segment (start 102.5525 85.4075) (end 101.71097 85.4075) (width 0.2) (layer "B.Cu") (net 3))
 (segment (start 95.6056 74.2696) (end 95.1992 73.8632) (width 0.2) (layer "B.Cu") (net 3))
 (segment (start 142.748 86.198) (end 146.85 90.3) (width 0.2) (layer "B.Cu") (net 3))
 (segment (start 112.0648 75.7936) (end 112.1309 75.7275) (width 0.2) (layer "B.Cu") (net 3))
 (segment (start 111.9625 94.8175) (end 116.4625 94.8175) (width 0.2) (layer "B.Cu") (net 3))
 (segment (start 97.45 89.66847) (end 97.45 94.755) (width 0.2) (layer "B.Cu") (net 3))
 (segment (start 112.1309 75.7275) (end 113.3856 75.7275) (width 0.2) (layer "B.Cu") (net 3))
 (segment (start 102.5525 85.4075) (end 110.4773 93.3323) (width 0.2) (layer "B.Cu") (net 3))
 (segment (start 134.85 90.3) (end 146.85 90.3) (width 0.2) (layer "B.Cu") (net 3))
 (segment (start 129.794 93.9292) (end 131.2208 93.9292) (width 0.2) (layer "B.Cu") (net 3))
 (segment (start 97.4125 75.7525) (end 97.0885 75.7525) (width 0.2) (layer "B.Cu") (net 3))
 (segment (start 111.9124 75.7174) (end 111.9124 75.7936) (width 0.2) (layer "B.Cu") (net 3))
 (segment (start 131.2208 93.9292) (end 132.35 92.8) (width 0.2) (layer "B.Cu") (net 3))
 (segment (start 101.71097 85.4075) (end 97.45 89.66847) (width 0.2) (layer "B.Cu") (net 3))
 (segment (start 121.6025 85.4075) (end 127.3048 91.1098) (width 0.2) (layer "B.Cu") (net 3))
 (segment (start 110.4773 93.3323) (end 111.9625 94.8175) (width 0.2) (layer "B.Cu") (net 3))
 (segment (start 95.6056 78.4606) (end 95.6056 74.2696) (width 0.2) (layer "B.Cu") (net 3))
 (segment (start 132.35 92.8) (end 134.85 90.3) (width 0.2) (layer "B.Cu") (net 3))
 (segment (start 112.83617 93.3323) (end 110.4773 93.3323) (width 0.2) (layer "B.Cu") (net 3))
 (segment (start 120.76097 85.4075) (end 112.83617 93.3323) (width 0.2) (layer "B.Cu") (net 3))
 (segment (start 102.5525 85.4075) (end 95.6056 78.4606) (width 0.2) (layer "B.Cu") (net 3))
 (segment (start 101.767684 66.3575) (end 102.5525 66.3575) (width 0.2) (layer "B.Cu") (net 3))
 (segment (start 111.9124 75.7936) (end 112.0648 75.7936) (width 0.2) (layer "B.Cu") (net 3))
 (segment (start 110.3376 78.7908) (end 110.3376 88.9) (width 0.2) (layer "F.Cu") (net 17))
 (segment (start 110.3376 88.9) (end 105.0036 94.234) (width 0.2) (layer "F.Cu") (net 17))
 (via (at 110.3376 78.7908) (size 0.6) (drill 0.3) (layers "F.Cu" "B.Cu") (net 17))
 (via (at 105.0036 94.234) (size 0.6) (drill 0.3) (layers "F.Cu" "B.Cu") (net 17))
 (segment (start 104.4826 94.755) (end 102.65 94.755) (width 0.2) (layer "B.Cu") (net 17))
 (segment (start 105.0036 94.234) (end 104.4826 94.755) (width 0.2) (layer "B.Cu") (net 17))
 (segment (start 116.4125 77.2275) (end 111.9009 77.2275) (width 0.2) (layer "B.Cu") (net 17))
 (segment (start 111.9009 77.2275) (end 110.3376 78.7908) (width 0.2) (layer "B.Cu") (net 17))
 (segment (start 106.350609 91.101637) (end 106.350609 79.120191) (width 0.2) (layer "F.Cu") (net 1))
 (segment (start 106.350609 79.120191) (end 106.4768 78.994) (width 0.2) (layer "F.Cu") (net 1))
 (via (at 106.350609 91.101637) (size 0.6) (drill 0.3) (layers "F.Cu" "B.Cu") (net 1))
 (via (at 106.4768 78.994) (size 0.6) (drill 0.3) (layers "F.Cu" "B.Cu") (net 1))
 (segment (start 106.4768 78.486) (end 107.1118 77.851) (width 0.2) (layer "B.Cu") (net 1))
 (segment (start 121.434904 77.442354) (end 121.413458 77.389794) (width 0.2) (layer "B.Cu") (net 1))
 (segment (start 106.5133 77.2525) (end 107.1118 77.851) (width 0.2) (layer "B.Cu") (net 1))
 (segment (start 121.413458 77.389794) (end 121.450206 77.389794) (width 0.2) (layer "B.Cu") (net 1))
 (segment (start 121.458058 77.4192) (end 121.434904 77.442354) (width 0.2) (layer "B.Cu") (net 1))
 (segment (start 103.832543 96.255) (end 106.233835 93.853708) (width 0.2) (layer "B.Cu") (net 1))
 (segment (start 106.290837 91.101637) (end 106.350609 91.101637) (width 0.2) (layer "B.Cu") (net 1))
 (segment (start 147.34 62.1) (end 144.941 59.701) (width 0.2) (layer "B.Cu") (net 1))
 (segment (start 122.627 97.282) (end 121.6625 96.3175) (width 0.2) (layer "B.Cu") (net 1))
 (segment (start 121.450206 77.389794) (end 121.6125 77.2275) (width 0.2) (layer "B.Cu") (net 1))
 (segment (start 106.233835 91.044635) (end 106.290837 91.101637) (width 0.2) (layer "B.Cu") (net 1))
 (segment (start 109.22 79.9592) (end 122.0724 79.9592) (width 0.2) (layer "B.Cu") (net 1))
 (segment (start 127.3556 59.701) (end 126.1872 60.8694) (width 0.2) (layer "B.Cu") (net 1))
 (segment (start 110.678127 98.298) (end 122.6312 98.298) (width 0.2) (layer "B.Cu") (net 1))
 (segment (start 102.65 96.255) (end 103.832543 96.255) (width 0.2) (layer "B.Cu") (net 1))
 (segment (start 122.6312 98.298) (end 123.2916 97.6376) (width 0.2) (layer "B.Cu") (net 1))
 (segment (start 123.2916 97.6376) (end 122.936 97.282) (width 0.2) (layer "B.Cu") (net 1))
 (segment (start 106.233835 93.853708) (end 110.678127 98.298) (width 0.2) (layer "B.Cu") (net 1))
 (segment (start 126.1872 60.8694) (end 126.1872 77.4192) (width 0.2) (layer "B.Cu") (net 1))
 (segment (start 106.233835 93.853708) (end 106.233835 91.044635) (width 0.2) (layer "B.Cu") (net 1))
 (segment (start 106.4768 78.994) (end 106.4768 78.486) (width 0.2) (layer "B.Cu") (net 1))
 (segment (start 122.0724 79.9592) (end 123.444 78.5876) (width 0.2) (layer "B.Cu") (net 1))
 (segment (start 144.941 59.701) (end 127.3556 59.701) (width 0.2) (layer "B.Cu") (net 1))
 (segment (start 123.444 77.4192) (end 121.458058 77.4192) (width 0.2) (layer "B.Cu") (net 1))
 (segment (start 122.936 97.282) (end 122.627 97.282) (width 0.2) (layer "B.Cu") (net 1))
 (segment (start 102.6125 77.2525) (end 106.5133 77.2525) (width 0.2) (layer "B.Cu") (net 1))
 (segment (start 107.1118 77.851) (end 109.22 79.9592) (width 0.2) (layer "B.Cu") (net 1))
 (segment (start 126.1872 77.4192) (end 123.444 77.4192) (width 0.2) (layer "B.Cu") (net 1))
 (segment (start 123.444 78.5876) (end 123.444 77.4192) (width 0.2) (layer "B.Cu") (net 1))
 (segment (start 148.552 76.012) (end 147.34 74.8) (width 0.2) (layer "B.Cu") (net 12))
 (segment (start 96.2025 68.8975) (end 94.878186 68.8975) (width 0.2) (layer "B.Cu") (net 12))
 (segment (start 97.6035 81.485586) (end 97.6035 88.527814) (width 0.2) (layer "B.Cu") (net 12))
 (segment (start 148.552 97.2267) (end 148.552 76.012) (width 0.2) (layer "B.Cu") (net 12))
 (segment (start 97.6035 88.527814) (end 96.782814 89.3485) (width 0.2) (layer "B.Cu") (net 12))
 (segment (start 96.782814 92.028086) (end 87.377 101.4339) (width 0.2) (layer "B.Cu") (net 12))
 (segment (start 96.782814 89.3485) (end 96.782814 92.028086) (width 0.2) (layer "B.Cu") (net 12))
 (segment (start 89.9468 73.828886) (end 97.6035 81.485586) (width 0.2) (layer "B.Cu") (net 12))
 (segment (start 87.377 101.4339) (end 88.6045 102.6614) (width 0.2) (layer "B.Cu") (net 12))
 (segment (start 94.878186 68.8975) (end 89.9468 73.828886) (width 0.2) (layer "B.Cu") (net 12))
 (segment (start 143.1173 102.6614) (end 148.552 97.2267) (width 0.2) (layer "B.Cu") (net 12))
 (segment (start 88.6045 102.6614) (end 143.1173 102.6614) (width 0.2) (layer "B.Cu") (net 12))
 (segment (start 86.976 91.0844) (end 86.976 101.6) (width 0.2) (layer "B.Cu") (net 13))
 (segment (start 86.976 101.6) (end 88.45 103.074) (width 0.2) (layer "B.Cu") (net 13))
 (segment (start 152.5402 72.26) (end 147.34 72.26) (width 0.2) (layer "B.Cu") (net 13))
 (segment (start 154.499 100.0598) (end 154.499 74.2188) (width 0.2) (layer "B.Cu") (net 13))
 (segment (start 151.638 102.9208) (end 154.499 100.0598) (width 0.2) (layer "B.Cu") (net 13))
 (segment (start 90.1129 87.9475) (end 86.976 91.0844) (width 0.2) (layer "B.Cu") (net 13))
 (segment (start 96.2025 87.9475) (end 90.1129 87.9475) (width 0.2) (layer "B.Cu") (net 13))
 (segment (start 88.45 103.074) (end 151.638 103.074) (width 0.2) (layer "B.Cu") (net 13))
 (segment (start 154.499 74.2188) (end 152.5402 72.26) (width 0.2) (layer "B.Cu") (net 13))
 (segment (start 151.638 103.074) (end 151.638 102.9208) (width 0.2) (layer "B.Cu") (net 13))
 (segment (start 126.1364 59.701) (end 128.524 62.0886) (width 0.2) (layer "F.Cu") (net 6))
 (segment (start 116.1796 59.701) (end 126.1364 59.701) (width 0.2) (layer "F.Cu") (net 6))
 (segment (start 115.2525 68.8975) (end 115.2525 60.6281) (width 0.2) (layer "F.Cu") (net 6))
 (segment (start 128.524 91.474) (end 132.35 95.3) (width 0.2) (layer "F.Cu") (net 6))
 (segment (start 128.524 62.0886) (end 128.524 91.474) (width 0.2) (layer "F.Cu") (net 6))
 (segment (start 115.2525 60.6281) (end 116.1796 59.701) (width 0.2) (layer "F.Cu") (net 6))
 (segment (start 143.689892 95.3) (end 148.151 90.838892) (width 0.2) (layer "B.Cu") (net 6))
 (segment (start 148.151 90.838892) (end 148.151 78.151) (width 0.2) (layer "B.Cu") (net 6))
 (segment (start 148.151 78.151) (end 147.34 77.34) (width 0.2) (layer "B.Cu") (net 6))
 (segment (start 132.35 95.3) (end 143.689892 95.3) (width 0.2) (layer "B.Cu") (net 6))
 (segment (start 143.5584 65.9384) (end 147.34 69.72) (width 0.2) (layer "F.Cu") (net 14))
 (segment (start 142.7988 65.9384) (end 143.5584 65.9384) (width 0.2) (layer "F.Cu") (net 14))
 (via (at 142.7988 65.9384) (size 0.6) (drill 0.3) (layers "F.Cu" "B.Cu") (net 14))
 (segment (start 127.9144 65.9384) (end 142.9512 65.9384) (width 0.2) (layer "B.Cu") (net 14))
 (segment (start 126.7038 77.549343) (end 126.7038 67.149) (width 0.2) (layer "B.Cu") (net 14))
 (segment (start 126.7038 67.149) (end 127.9144 65.9384) (width 0.2) (layer "B.Cu") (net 14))
 (segment (start 115.2525 87.9475) (end 116.305643 87.9475) (width 0.2) (layer "B.Cu") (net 14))
 (segment (start 116.305643 87.9475) (end 126.7038 77.549343) (width 0.2) (layer "B.Cu") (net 14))
 (segment (start 122.4527 94.8175) (end 121.6625 94.8175) (width 0.2) (layer "B.Cu") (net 16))
 (segment (start 97.45 99.736) (end 97.6884 99.9744) (width 0.2) (layer "B.Cu") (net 16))
 (segment (start 97.45 96.255) (end 97.45 99.736) (width 0.2) (layer "B.Cu") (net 16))
 (segment (start 127.1524 99.5172) (end 122.4527 94.8175) (width 0.2) (layer "B.Cu") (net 16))
 (segment (start 97.6884 99.9744) (end 98.1456 99.5172) (width 0.2) (layer "B.Cu") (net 16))
 (segment (start 98.1456 99.5172) (end 127.1524 99.5172) (width 0.2) (layer "B.Cu") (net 16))
 (segment (start 124.5108 82.1944) (end 125.6792 81.026) (width 0.2) (layer "F.Cu") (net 11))
 (segment (start 127.254 68.2752) (end 127.254 68.2244) (width 0.2) (layer "F.Cu") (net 11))
 (segment (start 125.6792 81.026) (end 125.6792 69.85) (width 0.2) (layer "F.Cu") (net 11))
 (segment (start 109.5756 95.7072) (end 111.506 93.7768) (width 0.2) (layer "F.Cu") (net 11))
 (segment (start 111.506 93.7768) (end 111.506 82.1944) (width 0.2) (layer "F.Cu") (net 11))
 (segment (start 125.6792 69.85) (end 127.254 68.2752) (width 0.2) (layer "F.Cu") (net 11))
 (segment (start 127.254 68.2244) (end 127.3048 68.1736) (width 0.2) (layer "F.Cu") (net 11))
 (segment (start 111.506 82.1944) (end 124.5108 82.1944) (width 0.2) (layer "F.Cu") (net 11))
 (via (at 109.5756 95.7072) (size 0.6) (drill 0.3) (layers "F.Cu" "B.Cu") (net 11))
 (via (at 127.3048 68.1736) (size 0.6) (drill 0.3) (layers "F.Cu" "B.Cu") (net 11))
 (segment (start 116.4625 96.3175) (end 110.1859 96.3175) (width 0.2) (layer "B.Cu") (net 11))
 (segment (start 127.3048 68.1736) (end 127.7112 68.58) (width 0.2) (layer "B.Cu") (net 11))
 (segment (start 134.112 70.248) (end 132.1 72.26) (width 0.2) (layer "B.Cu") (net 11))
 (segment (start 110.1859 96.3175) (end 109.5756 95.7072) (width 0.2) (layer "B.Cu") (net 11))
 (segment (start 127.7112 68.58) (end 134.112 68.58) (width 0.2) (layer "B.Cu") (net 11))
 (segment (start 134.112 68.58) (end 134.112 70.248) (width 0.2) (layer "B.Cu") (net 11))
 (segment (start 132.35 90.3) (end 132.35 77.59) (width 0.2) (layer "B.Cu") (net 5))
 (segment (start 132.1 77.34) (end 132.1 74.8) (width 0.2) (layer "B.Cu") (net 5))
 (segment (start 132.35 77.59) (end 132.1 77.34) (width 0.2) (layer "B.Cu") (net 5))
 (segment (start 132.1 69.72) (end 129.7208 69.72) (width 0.2) (layer "B.Cu") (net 7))
 (segment (start 129.5908 102.2604) (end 142.9512 102.2604) (width 0.2) (layer "B.Cu") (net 7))
 (segment (start 129.7208 69.72) (end 128.4224 71.0184) (width 0.2) (layer "B.Cu") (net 7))
 (segment (start 142.9512 102.2604) (end 146.85 98.3616) (width 0.2) (layer "B.Cu") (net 7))
 (segment (start 128.4224 101.092) (end 129.5908 102.2604) (width 0.2) (layer "B.Cu") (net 7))
 (segment (start 128.4224 71.0184) (end 128.4224 101.092) (width 0.2) (layer "B.Cu") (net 7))
 (segment (start 146.85 98.3616) (end 146.85 95.3) (width 0.2) (layer "B.Cu") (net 7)))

